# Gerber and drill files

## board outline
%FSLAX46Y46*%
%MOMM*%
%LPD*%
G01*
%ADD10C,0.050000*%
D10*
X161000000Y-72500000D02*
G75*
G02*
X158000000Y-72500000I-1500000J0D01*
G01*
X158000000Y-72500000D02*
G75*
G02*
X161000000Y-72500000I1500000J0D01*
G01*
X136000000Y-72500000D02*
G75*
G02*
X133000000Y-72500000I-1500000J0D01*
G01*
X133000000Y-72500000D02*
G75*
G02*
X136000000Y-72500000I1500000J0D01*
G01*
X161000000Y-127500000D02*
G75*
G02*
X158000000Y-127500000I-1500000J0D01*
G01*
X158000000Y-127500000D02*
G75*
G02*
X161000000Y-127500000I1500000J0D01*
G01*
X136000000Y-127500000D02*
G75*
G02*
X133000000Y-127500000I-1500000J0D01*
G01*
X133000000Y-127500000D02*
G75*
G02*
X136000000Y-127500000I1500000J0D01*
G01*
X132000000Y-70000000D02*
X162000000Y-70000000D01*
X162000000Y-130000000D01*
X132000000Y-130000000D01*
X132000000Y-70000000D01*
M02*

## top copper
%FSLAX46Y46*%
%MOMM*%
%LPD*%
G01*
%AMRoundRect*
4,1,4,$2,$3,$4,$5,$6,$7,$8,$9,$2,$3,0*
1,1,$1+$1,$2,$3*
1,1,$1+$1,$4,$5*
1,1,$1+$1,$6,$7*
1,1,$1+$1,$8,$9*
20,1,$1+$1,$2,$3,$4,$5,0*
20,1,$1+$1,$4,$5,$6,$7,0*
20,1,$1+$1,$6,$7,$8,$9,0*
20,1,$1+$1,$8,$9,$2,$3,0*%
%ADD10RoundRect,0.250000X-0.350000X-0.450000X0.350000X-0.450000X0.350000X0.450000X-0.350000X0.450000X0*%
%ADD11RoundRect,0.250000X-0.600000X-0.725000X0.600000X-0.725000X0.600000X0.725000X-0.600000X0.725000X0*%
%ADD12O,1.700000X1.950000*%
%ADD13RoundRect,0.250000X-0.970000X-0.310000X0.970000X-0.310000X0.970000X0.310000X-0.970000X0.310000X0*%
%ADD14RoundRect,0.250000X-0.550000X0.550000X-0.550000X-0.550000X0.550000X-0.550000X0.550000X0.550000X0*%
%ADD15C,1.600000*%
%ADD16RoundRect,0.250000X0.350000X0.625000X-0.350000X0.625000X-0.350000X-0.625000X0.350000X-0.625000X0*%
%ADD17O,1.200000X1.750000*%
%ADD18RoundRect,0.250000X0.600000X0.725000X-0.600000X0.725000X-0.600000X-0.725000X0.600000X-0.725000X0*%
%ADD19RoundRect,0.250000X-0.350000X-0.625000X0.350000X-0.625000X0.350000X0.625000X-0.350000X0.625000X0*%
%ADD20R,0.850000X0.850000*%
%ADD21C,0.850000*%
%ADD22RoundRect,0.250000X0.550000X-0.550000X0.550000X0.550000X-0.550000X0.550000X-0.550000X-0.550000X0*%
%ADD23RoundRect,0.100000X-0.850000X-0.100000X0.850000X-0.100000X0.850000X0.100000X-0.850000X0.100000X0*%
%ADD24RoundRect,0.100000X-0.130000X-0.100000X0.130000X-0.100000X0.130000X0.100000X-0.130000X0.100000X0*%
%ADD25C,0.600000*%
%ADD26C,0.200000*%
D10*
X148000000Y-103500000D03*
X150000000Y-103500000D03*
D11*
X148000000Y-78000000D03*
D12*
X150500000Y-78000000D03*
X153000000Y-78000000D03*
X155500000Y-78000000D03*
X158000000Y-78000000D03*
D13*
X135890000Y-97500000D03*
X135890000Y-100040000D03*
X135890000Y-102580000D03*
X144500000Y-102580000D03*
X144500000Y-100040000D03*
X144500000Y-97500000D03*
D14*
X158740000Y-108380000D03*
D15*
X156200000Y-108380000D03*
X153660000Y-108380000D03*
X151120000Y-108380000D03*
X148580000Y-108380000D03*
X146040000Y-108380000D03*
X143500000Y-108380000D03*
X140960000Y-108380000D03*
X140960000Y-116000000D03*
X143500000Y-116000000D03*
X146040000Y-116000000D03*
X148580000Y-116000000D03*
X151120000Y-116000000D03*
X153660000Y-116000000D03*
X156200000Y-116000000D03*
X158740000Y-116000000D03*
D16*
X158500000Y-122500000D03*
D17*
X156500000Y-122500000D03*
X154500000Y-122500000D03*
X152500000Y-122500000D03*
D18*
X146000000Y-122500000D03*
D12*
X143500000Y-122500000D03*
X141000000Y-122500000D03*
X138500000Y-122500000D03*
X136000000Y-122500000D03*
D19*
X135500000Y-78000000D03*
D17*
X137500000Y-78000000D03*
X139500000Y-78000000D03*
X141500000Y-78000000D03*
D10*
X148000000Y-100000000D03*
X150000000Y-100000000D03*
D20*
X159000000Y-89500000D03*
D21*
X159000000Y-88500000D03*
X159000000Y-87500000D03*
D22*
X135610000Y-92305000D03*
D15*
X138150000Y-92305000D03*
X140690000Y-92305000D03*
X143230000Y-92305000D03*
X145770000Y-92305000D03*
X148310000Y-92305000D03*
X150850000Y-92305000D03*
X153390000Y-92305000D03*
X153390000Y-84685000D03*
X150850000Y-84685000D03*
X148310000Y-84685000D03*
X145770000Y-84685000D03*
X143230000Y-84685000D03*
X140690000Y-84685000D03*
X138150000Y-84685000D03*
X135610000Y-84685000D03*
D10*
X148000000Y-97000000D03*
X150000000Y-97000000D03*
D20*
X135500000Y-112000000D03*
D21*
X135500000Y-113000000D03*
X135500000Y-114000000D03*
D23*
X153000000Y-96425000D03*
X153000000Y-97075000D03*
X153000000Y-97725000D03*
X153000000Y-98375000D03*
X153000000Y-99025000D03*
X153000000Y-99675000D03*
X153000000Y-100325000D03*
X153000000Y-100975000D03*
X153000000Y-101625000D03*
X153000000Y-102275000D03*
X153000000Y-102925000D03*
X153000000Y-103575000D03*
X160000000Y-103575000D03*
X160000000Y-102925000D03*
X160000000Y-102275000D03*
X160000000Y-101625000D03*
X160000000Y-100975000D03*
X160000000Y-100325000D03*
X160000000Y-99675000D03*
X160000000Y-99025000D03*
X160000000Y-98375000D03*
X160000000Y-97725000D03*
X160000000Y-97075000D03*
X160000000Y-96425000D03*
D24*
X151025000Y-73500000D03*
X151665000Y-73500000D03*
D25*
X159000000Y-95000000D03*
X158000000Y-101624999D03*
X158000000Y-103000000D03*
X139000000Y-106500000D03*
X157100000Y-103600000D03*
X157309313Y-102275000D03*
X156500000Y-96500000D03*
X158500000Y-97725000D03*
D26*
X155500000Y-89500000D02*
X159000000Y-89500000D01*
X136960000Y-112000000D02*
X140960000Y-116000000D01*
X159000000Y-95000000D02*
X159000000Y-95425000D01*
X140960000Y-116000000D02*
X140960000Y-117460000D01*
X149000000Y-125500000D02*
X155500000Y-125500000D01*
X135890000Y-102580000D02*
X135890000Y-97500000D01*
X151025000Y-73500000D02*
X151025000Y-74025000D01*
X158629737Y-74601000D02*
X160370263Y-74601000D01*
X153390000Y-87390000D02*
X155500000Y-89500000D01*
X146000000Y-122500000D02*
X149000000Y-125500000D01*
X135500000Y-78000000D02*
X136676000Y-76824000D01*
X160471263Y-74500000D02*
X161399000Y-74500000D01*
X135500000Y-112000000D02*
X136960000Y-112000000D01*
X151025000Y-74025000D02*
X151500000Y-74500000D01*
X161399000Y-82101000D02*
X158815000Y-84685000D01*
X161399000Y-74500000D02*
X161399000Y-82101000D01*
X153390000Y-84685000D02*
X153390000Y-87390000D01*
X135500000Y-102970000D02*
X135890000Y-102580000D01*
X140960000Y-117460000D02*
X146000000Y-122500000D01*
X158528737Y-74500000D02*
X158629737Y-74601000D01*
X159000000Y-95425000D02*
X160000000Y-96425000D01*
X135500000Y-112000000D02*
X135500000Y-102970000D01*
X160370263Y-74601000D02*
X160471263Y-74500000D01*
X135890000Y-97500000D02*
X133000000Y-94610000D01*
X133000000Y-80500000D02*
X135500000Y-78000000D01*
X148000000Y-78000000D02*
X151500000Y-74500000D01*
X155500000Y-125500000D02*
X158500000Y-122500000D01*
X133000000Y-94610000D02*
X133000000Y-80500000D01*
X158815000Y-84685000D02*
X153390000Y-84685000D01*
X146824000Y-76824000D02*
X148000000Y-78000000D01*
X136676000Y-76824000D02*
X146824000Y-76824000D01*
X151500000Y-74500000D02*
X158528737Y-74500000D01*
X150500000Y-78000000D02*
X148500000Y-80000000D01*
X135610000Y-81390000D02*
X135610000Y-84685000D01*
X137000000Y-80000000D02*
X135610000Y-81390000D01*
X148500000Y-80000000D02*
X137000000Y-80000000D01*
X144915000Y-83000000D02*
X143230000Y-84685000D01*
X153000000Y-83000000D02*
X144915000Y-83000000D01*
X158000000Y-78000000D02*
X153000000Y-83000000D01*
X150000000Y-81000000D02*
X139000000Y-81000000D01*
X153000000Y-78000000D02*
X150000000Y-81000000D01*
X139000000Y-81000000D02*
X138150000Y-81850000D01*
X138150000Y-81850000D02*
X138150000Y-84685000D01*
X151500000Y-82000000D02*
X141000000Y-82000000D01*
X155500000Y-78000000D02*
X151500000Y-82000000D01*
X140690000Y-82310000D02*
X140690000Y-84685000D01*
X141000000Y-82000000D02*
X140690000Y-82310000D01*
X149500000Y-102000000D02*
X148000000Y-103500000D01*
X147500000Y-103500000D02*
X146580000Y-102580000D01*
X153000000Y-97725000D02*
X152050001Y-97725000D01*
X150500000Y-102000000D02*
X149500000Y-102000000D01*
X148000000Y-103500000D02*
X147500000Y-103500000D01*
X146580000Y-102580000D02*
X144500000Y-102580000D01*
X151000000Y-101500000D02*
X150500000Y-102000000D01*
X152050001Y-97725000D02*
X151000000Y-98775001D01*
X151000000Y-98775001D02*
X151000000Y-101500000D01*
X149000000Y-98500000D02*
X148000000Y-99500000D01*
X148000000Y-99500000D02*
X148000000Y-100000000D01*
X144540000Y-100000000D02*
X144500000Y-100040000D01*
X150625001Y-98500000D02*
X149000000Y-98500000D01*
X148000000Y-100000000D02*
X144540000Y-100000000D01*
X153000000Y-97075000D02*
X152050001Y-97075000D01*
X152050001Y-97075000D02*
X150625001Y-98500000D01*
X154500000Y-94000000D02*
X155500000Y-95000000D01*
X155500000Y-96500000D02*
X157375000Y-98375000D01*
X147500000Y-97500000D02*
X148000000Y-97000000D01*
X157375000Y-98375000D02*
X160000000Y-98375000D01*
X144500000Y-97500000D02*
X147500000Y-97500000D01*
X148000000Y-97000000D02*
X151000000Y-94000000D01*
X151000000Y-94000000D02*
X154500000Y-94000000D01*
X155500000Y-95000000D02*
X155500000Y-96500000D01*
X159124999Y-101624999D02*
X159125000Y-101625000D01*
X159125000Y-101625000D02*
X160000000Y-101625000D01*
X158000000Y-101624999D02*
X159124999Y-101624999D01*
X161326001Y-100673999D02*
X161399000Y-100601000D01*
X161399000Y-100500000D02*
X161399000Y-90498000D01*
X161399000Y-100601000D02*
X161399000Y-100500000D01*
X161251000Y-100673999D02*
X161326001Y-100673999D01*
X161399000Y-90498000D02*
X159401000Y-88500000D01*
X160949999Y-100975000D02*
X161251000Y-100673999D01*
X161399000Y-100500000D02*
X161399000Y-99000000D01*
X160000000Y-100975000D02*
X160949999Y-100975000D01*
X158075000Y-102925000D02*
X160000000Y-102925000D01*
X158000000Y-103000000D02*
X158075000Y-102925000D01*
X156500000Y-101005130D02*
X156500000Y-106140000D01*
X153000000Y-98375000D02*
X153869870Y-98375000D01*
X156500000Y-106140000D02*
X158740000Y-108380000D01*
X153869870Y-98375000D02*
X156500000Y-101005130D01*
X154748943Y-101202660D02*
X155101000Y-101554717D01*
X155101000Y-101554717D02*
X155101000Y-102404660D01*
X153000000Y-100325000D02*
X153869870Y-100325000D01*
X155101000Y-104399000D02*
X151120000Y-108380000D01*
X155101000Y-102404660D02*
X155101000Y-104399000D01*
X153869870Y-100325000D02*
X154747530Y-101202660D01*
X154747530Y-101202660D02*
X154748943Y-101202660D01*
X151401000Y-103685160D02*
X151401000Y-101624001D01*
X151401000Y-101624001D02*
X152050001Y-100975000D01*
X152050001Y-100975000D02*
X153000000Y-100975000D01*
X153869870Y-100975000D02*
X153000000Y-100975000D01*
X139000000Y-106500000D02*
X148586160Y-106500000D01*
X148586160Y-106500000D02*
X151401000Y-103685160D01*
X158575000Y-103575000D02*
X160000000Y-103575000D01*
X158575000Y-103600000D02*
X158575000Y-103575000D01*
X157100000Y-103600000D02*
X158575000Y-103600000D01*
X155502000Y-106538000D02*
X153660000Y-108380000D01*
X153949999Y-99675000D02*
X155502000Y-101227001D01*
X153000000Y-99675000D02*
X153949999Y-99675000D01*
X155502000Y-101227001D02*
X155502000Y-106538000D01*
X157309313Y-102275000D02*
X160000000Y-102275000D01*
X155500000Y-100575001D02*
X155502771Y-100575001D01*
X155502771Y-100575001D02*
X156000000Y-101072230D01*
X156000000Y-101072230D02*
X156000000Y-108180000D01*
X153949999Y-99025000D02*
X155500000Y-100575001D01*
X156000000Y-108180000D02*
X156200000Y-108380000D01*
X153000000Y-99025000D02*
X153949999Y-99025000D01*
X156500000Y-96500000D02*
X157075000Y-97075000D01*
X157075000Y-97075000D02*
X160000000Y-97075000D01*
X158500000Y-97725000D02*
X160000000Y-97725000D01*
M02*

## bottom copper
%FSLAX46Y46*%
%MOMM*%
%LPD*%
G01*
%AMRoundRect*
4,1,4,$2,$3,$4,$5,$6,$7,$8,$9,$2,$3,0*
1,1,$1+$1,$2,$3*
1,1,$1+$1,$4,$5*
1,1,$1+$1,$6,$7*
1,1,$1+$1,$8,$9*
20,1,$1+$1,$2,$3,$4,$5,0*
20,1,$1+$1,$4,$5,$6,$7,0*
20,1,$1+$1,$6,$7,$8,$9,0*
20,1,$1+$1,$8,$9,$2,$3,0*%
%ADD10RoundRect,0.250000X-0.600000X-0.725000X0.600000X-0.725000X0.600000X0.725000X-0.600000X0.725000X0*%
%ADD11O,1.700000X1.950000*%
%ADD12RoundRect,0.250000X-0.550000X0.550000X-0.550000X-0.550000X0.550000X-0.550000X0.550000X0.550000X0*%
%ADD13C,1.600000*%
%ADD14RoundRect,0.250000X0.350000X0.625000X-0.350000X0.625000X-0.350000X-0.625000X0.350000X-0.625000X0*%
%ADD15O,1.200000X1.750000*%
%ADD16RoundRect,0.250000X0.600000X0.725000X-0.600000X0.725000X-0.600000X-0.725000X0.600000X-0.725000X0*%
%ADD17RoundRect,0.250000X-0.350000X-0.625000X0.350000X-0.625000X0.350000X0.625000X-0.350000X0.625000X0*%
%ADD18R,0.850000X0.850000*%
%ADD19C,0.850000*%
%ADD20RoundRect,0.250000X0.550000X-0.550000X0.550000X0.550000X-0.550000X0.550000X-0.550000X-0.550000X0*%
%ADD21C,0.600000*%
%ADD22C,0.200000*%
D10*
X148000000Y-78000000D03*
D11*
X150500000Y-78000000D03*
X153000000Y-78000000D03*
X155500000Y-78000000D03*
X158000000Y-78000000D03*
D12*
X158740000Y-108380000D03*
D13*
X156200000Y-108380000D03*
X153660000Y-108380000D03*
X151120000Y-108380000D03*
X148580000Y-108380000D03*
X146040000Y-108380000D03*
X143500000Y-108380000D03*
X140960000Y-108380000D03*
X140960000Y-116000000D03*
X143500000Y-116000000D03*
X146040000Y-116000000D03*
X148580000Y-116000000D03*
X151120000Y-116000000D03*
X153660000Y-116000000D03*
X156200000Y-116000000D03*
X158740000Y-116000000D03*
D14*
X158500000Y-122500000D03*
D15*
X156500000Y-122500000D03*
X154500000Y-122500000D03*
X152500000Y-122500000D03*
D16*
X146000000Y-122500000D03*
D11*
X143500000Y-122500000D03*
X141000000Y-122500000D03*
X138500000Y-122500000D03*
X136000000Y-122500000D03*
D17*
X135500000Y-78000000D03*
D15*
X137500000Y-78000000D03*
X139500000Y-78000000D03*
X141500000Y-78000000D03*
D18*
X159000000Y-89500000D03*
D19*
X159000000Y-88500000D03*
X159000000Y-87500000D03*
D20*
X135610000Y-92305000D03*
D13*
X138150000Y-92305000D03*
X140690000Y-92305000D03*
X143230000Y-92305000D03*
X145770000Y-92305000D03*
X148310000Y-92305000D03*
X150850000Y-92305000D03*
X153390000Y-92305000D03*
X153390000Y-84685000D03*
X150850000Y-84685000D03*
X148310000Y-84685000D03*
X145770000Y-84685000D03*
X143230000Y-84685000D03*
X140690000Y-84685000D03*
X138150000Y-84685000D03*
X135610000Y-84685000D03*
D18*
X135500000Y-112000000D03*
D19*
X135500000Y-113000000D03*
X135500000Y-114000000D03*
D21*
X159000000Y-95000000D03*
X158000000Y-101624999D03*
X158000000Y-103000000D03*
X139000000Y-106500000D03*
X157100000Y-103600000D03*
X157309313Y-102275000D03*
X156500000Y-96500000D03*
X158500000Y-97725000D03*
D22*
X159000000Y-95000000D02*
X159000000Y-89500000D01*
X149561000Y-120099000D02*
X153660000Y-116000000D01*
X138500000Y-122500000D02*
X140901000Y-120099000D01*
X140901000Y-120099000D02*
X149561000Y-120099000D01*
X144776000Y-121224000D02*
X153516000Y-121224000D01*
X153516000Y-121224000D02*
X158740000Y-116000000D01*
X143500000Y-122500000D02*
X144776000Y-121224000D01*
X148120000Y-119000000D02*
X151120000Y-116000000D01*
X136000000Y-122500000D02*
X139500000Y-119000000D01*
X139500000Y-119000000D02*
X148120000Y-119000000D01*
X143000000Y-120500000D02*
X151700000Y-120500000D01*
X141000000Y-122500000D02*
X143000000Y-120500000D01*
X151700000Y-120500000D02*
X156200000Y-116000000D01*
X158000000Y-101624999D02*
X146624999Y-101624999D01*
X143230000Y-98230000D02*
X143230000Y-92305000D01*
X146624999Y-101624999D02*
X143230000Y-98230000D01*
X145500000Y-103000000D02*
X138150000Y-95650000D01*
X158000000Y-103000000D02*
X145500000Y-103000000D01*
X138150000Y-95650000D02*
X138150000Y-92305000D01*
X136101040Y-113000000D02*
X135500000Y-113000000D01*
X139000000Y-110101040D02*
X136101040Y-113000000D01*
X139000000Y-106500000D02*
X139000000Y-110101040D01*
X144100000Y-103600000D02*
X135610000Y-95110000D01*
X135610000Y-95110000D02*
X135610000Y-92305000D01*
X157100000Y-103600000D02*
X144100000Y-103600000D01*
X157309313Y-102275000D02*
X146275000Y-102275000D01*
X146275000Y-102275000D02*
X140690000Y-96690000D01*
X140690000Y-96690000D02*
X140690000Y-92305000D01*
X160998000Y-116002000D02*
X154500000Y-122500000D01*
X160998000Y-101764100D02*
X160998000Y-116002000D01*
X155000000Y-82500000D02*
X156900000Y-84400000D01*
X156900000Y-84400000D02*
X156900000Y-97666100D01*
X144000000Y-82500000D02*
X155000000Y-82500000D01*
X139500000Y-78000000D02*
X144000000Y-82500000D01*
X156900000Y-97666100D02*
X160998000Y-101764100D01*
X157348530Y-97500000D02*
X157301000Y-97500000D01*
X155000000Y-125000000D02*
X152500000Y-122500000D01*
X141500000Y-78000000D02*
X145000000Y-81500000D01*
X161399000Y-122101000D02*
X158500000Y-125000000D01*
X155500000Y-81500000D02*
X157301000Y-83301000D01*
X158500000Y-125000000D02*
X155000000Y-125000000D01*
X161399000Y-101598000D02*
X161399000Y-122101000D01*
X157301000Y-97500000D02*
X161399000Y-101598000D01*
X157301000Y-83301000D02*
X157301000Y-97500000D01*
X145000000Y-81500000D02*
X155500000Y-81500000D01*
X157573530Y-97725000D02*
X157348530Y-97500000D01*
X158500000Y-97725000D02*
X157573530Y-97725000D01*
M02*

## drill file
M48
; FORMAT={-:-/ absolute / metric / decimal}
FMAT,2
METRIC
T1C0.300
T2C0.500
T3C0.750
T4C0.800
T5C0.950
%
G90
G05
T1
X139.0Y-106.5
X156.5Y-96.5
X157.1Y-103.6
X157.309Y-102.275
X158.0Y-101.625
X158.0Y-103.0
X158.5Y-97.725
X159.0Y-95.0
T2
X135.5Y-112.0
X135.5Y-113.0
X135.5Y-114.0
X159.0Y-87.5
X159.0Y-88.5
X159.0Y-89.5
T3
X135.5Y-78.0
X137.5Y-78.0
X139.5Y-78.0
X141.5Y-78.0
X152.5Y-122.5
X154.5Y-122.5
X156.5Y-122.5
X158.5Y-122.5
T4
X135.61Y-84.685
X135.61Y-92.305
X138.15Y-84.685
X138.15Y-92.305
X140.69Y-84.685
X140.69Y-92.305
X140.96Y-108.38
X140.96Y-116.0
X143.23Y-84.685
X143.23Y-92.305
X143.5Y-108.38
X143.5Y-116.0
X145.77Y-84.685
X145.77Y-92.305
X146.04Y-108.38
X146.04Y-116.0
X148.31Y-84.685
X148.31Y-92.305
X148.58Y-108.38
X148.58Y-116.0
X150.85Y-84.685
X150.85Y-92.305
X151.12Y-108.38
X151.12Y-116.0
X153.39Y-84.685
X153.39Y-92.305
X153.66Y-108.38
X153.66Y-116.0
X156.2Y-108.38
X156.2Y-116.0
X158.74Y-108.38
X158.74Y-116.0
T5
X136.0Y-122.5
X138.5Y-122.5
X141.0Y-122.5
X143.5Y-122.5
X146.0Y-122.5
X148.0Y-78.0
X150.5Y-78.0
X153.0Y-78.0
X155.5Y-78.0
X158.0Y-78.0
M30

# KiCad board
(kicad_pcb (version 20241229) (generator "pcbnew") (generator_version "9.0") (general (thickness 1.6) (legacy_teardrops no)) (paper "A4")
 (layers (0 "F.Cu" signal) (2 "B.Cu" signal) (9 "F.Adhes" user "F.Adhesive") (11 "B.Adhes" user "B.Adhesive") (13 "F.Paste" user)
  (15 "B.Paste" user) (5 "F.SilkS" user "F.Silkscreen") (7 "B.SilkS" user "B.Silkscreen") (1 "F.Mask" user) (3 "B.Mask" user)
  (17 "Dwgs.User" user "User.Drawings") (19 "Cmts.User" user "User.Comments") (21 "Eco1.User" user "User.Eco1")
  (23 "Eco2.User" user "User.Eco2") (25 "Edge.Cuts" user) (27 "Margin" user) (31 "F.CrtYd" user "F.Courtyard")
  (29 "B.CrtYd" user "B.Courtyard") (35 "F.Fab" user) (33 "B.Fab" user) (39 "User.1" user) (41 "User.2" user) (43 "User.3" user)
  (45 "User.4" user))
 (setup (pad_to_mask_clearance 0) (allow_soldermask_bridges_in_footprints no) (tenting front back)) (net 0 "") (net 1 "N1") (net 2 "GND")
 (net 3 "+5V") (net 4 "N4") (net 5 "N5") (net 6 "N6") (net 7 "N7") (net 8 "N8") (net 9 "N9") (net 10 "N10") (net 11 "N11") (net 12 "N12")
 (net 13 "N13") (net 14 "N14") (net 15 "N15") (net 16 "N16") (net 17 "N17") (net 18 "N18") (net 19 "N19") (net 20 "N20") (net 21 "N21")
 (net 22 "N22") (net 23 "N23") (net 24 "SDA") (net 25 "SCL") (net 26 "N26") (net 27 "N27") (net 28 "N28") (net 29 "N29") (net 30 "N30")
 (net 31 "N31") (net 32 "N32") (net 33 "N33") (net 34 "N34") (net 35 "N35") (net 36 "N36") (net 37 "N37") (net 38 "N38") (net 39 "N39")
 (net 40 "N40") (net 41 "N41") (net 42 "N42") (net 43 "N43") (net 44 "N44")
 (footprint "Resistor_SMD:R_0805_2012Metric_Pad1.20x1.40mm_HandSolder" (layer "F.Cu") (at 149 103.5)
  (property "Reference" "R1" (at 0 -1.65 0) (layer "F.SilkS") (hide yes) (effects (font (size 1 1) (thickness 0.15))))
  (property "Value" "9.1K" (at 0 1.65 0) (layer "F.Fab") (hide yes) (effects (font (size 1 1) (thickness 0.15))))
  (pad "1" smd roundrect (at -1 0) (size 1.2 1.4) (layers "F.Cu" "F.Mask" "F.Paste") (roundrect_rratio 0.208333) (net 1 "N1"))
  (pad "2" smd roundrect (at 1 0) (size 1.2 1.4) (layers "F.Cu" "F.Mask" "F.Paste") (roundrect_rratio 0.208333) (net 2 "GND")))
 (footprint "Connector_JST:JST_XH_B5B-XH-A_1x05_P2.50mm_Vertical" (layer "F.Cu") (at 148 78)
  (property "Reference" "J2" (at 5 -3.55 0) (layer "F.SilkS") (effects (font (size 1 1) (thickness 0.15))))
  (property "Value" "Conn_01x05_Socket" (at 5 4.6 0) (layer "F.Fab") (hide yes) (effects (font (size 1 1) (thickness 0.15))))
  (pad "1" thru_hole roundrect (at 0 0) (size 1.7 1.95) (drill 0.95) (layers "*.Cu" "*.Mask") (remove_unused_layers no)
   (roundrect_rratio 0.147059) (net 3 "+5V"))
  (pad "2" thru_hole oval (at 2.5 0) (size 1.7 1.95) (drill 0.95) (layers "*.Cu" "*.Mask") (remove_unused_layers no) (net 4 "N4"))
  (pad "3" thru_hole oval (at 5 0) (size 1.7 1.95) (drill 0.95) (layers "*.Cu" "*.Mask") (remove_unused_layers no) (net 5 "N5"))
  (pad "4" thru_hole oval (at 7.5 0) (size 1.7 1.95) (drill 0.95) (layers "*.Cu" "*.Mask") (remove_unused_layers no) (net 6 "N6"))
  (pad "5" thru_hole oval (at 10 0) (size 1.7 1.95) (drill 0.95) (layers "*.Cu" "*.Mask") (remove_unused_layers no) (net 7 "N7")))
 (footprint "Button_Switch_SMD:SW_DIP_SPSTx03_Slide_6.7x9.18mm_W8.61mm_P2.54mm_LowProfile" (layer "F.Cu") (at 140.195 100.04)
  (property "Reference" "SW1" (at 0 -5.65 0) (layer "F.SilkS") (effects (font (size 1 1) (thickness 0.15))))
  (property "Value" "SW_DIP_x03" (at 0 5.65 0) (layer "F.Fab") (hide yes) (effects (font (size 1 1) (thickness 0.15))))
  (pad "1" smd roundrect (at -4.305 -2.54) (size 2.44 1.12) (layers "F.Cu" "F.Mask" "F.Paste") (roundrect_rratio 0.223214) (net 3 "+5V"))
  (pad "2" smd roundrect (at -4.305 0) (size 2.44 1.12) (layers "F.Cu" "F.Mask" "F.Paste") (roundrect_rratio 0.223214) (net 3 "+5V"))
  (pad "3" smd roundrect (at -4.305 2.54) (size 2.44 1.12) (layers "F.Cu" "F.Mask" "F.Paste") (roundrect_rratio 0.223214) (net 3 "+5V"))
  (pad "4" smd roundrect (at 4.305 2.54) (size 2.44 1.12) (layers "F.Cu" "F.Mask" "F.Paste") (roundrect_rratio 0.223214) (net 1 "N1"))
  (pad "5" smd roundrect (at 4.305 0) (size 2.44 1.12) (layers "F.Cu" "F.Mask" "F.Paste") (roundrect_rratio 0.223214) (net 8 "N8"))
  (pad "6" smd roundrect (at 4.305 -2.54) (size 2.44 1.12) (layers "F.Cu" "F.Mask" "F.Paste") (roundrect_rratio 0.223214) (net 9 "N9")))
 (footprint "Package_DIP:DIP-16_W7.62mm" (layer "F.Cu") (at 158.74 108.38 -90)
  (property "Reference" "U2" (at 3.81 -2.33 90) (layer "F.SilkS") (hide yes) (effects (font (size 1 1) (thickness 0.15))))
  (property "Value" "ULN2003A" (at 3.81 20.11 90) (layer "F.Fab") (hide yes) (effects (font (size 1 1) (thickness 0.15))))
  (pad "1" thru_hole roundrect (at 0 0 270) (size 1.6 1.6) (drill 0.8) (layers "*.Cu" "*.Mask") (remove_unused_layers no)
   (roundrect_rratio 0.15625) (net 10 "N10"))
  (pad "2" thru_hole circle (at 0 2.54 270) (size 1.6 1.6) (drill 0.8) (layers "*.Cu" "*.Mask") (remove_unused_layers no) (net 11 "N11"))
  (pad "3" thru_hole circle (at 0 5.08 270) (size 1.6 1.6) (drill 0.8) (layers "*.Cu" "*.Mask") (remove_unused_layers no) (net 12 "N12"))
  (pad "4" thru_hole circle (at 0 7.62 270) (size 1.6 1.6) (drill 0.8) (layers "*.Cu" "*.Mask") (remove_unused_layers no) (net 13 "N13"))
  (pad "5" thru_hole circle (at 0 10.16 270) (size 1.6 1.6) (drill 0.8) (layers "*.Cu" "*.Mask") (remove_unused_layers no) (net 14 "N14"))
  (pad "6" thru_hole circle (at 0 12.7 270) (size 1.6 1.6) (drill 0.8) (layers "*.Cu" "*.Mask") (remove_unused_layers no) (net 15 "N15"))
  (pad "7" thru_hole circle (at 0 15.24 270) (size 1.6 1.6) (drill 0.8) (layers "*.Cu" "*.Mask") (remove_unused_layers no) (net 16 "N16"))
  (pad "8" thru_hole circle (at 0 17.78 270) (size 1.6 1.6) (drill 0.8) (layers "*.Cu" "*.Mask") (remove_unused_layers no) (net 2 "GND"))
  (pad "9" thru_hole circle (at 7.62 17.78 270) (size 1.6 1.6) (drill 0.8) (layers "*.Cu" "*.Mask") (remove_unused_layers no) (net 3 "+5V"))
  (pad "10" thru_hole circle (at 7.62 15.24 270) (size 1.6 1.6) (drill 0.8) (layers "*.Cu" "*.Mask") (remove_unused_layers no)
   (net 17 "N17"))
  (pad "11" thru_hole circle (at 7.62 12.7 270) (size 1.6 1.6) (drill 0.8) (layers "*.Cu" "*.Mask") (remove_unused_layers no) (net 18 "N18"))
  (pad "12" thru_hole circle (at 7.62 10.16 270) (size 1.6 1.6) (drill 0.8) (layers "*.Cu" "*.Mask") (remove_unused_layers no)
   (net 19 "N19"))
  (pad "13" thru_hole circle (at 7.62 7.62 270) (size 1.6 1.6) (drill 0.8) (layers "*.Cu" "*.Mask") (remove_unused_layers no) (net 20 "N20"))
  (pad "14" thru_hole circle (at 7.62 5.08 270) (size 1.6 1.6) (drill 0.8) (layers "*.Cu" "*.Mask") (remove_unused_layers no) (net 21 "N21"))
  (pad "15" thru_hole circle (at 7.62 2.54 270) (size 1.6 1.6) (drill 0.8) (layers "*.Cu" "*.Mask") (remove_unused_layers no) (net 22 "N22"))
  (pad "16" thru_hole circle (at 7.62 0 270) (size 1.6 1.6) (drill 0.8) (layers "*.Cu" "*.Mask") (remove_unused_layers no) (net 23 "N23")))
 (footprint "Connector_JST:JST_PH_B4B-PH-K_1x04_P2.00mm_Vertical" (layer "F.Cu") (at 158.5 122.5 180)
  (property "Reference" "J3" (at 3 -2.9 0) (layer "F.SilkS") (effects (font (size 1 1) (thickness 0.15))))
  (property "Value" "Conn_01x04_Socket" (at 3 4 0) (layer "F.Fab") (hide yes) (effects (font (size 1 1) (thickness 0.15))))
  (pad "1" thru_hole roundrect (at 0 0 180) (size 1.2 1.75) (drill 0.75) (layers "*.Cu" "*.Mask") (remove_unused_layers no)
   (roundrect_rratio 0.208333) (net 3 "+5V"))
  (pad "2" thru_hole oval (at 2 0 180) (size 1.2 1.75) (drill 0.75) (layers "*.Cu" "*.Mask") (remove_unused_layers no) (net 2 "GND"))
  (pad "3" thru_hole oval (at 4 0 180) (size 1.2 1.75) (drill 0.75) (layers "*.Cu" "*.Mask") (remove_unused_layers no) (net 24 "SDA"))
  (pad "4" thru_hole oval (at 6 0 180) (size 1.2 1.75) (drill 0.75) (layers "*.Cu" "*.Mask") (remove_unused_layers no) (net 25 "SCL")))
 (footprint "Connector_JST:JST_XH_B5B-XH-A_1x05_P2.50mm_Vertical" (layer "F.Cu") (at 146 122.5 180)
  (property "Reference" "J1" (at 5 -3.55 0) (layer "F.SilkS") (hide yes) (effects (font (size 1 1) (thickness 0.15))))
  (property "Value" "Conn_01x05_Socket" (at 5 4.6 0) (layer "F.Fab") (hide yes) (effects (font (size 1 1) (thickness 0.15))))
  (pad "1" thru_hole roundrect (at 0 0 180) (size 1.7 1.95) (drill 0.95) (layers "*.Cu" "*.Mask") (remove_unused_layers no)
   (roundrect_rratio 0.147059) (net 3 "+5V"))
  (pad "2" thru_hole oval (at 2.5 0 180) (size 1.7 1.95) (drill 0.95) (layers "*.Cu" "*.Mask") (remove_unused_layers no) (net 23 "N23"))
  (pad "3" thru_hole oval (at 5 0 180) (size 1.7 1.95) (drill 0.95) (layers "*.Cu" "*.Mask") (remove_unused_layers no) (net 22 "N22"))
  (pad "4" thru_hole oval (at 7.5 0 180) (size 1.7 1.95) (drill 0.95) (layers "*.Cu" "*.Mask") (remove_unused_layers no) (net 21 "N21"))
  (pad "5" thru_hole oval (at 10 0 180) (size 1.7 1.95) (drill 0.95) (layers "*.Cu" "*.Mask") (remove_unused_layers no) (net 20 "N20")))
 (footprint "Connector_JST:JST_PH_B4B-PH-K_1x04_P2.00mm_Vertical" (layer "F.Cu") (at 135.5 78)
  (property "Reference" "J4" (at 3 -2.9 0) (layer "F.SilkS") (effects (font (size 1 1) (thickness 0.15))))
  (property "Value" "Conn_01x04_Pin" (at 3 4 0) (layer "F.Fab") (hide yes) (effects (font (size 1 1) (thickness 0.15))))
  (pad "1" thru_hole roundrect (at 0 0) (size 1.2 1.75) (drill 0.75) (layers "*.Cu" "*.Mask") (remove_unused_layers no)
   (roundrect_rratio 0.208333) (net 3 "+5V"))
  (pad "2" thru_hole oval (at 2 0) (size 1.2 1.75) (drill 0.75) (layers "*.Cu" "*.Mask") (remove_unused_layers no) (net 2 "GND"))
  (pad "3" thru_hole oval (at 4 0) (size 1.2 1.75) (drill 0.75) (layers "*.Cu" "*.Mask") (remove_unused_layers no) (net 24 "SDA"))
  (pad "4" thru_hole oval (at 6 0) (size 1.2 1.75) (drill 0.75) (layers "*.Cu" "*.Mask") (remove_unused_layers no) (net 25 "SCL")))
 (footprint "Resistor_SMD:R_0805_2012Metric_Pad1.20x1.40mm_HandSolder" (layer "F.Cu") (at 149 100)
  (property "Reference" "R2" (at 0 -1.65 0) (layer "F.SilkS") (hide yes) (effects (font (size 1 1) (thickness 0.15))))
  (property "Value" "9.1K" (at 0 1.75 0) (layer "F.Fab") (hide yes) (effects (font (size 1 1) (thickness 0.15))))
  (pad "1" smd roundrect (at -1 0) (size 1.2 1.4) (layers "F.Cu" "F.Mask" "F.Paste") (roundrect_rratio 0.208333) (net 8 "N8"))
  (pad "2" smd roundrect (at 1 0) (size 1.2 1.4) (layers "F.Cu" "F.Mask" "F.Paste") (roundrect_rratio 0.208333) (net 2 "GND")))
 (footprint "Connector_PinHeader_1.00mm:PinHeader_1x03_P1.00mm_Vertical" (layer "F.Cu") (at 159 89.5 180)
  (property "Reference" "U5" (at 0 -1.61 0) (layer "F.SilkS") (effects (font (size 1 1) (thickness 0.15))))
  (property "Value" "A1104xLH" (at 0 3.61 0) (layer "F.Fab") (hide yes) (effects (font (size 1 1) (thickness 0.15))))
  (pad "1" thru_hole rect (at 0 0 180) (size 0.85 0.85) (drill 0.5) (layers "*.Cu" "*.Mask") (remove_unused_layers no) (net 3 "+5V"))
  (pad "2" thru_hole circle (at 0 1 180) (size 0.85 0.85) (drill 0.5) (layers "*.Cu" "*.Mask") (remove_unused_layers no) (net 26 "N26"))
  (pad "3" thru_hole circle (at 0 2 180) (size 0.85 0.85) (drill 0.5) (layers "*.Cu" "*.Mask") (remove_unused_layers no) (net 2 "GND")))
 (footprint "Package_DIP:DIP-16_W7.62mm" (layer "F.Cu") (at 135.61 92.305 90)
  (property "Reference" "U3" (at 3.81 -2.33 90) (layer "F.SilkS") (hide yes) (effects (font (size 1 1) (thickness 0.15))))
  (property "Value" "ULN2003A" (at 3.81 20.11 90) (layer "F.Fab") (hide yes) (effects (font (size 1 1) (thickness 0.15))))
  (pad "1" thru_hole roundrect (at 0 0 90) (size 1.6 1.6) (drill 0.8) (layers "*.Cu" "*.Mask") (remove_unused_layers no)
   (roundrect_rratio 0.15625) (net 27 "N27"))
  (pad "2" thru_hole circle (at 0 2.54 90) (size 1.6 1.6) (drill 0.8) (layers "*.Cu" "*.Mask") (remove_unused_layers no) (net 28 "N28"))
  (pad "3" thru_hole circle (at 0 5.08 90) (size 1.6 1.6) (drill 0.8) (layers "*.Cu" "*.Mask") (remove_unused_layers no) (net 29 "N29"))
  (pad "4" thru_hole circle (at 0 7.62 90) (size 1.6 1.6) (drill 0.8) (layers "*.Cu" "*.Mask") (remove_unused_layers no) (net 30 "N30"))
  (pad "5" thru_hole circle (at 0 10.16 90) (size 1.6 1.6) (drill 0.8) (layers "*.Cu" "*.Mask") (remove_unused_layers no) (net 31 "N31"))
  (pad "6" thru_hole circle (at 0 12.7 90) (size 1.6 1.6) (drill 0.8) (layers "*.Cu" "*.Mask") (remove_unused_layers no) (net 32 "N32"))
  (pad "7" thru_hole circle (at 0 15.24 90) (size 1.6 1.6) (drill 0.8) (layers "*.Cu" "*.Mask") (remove_unused_layers no) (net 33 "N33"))
  (pad "8" thru_hole circle (at 0 17.78 90) (size 1.6 1.6) (drill 0.8) (layers "*.Cu" "*.Mask") (remove_unused_layers no) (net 2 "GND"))
  (pad "9" thru_hole circle (at 7.62 17.78 90) (size 1.6 1.6) (drill 0.8) (layers "*.Cu" "*.Mask") (remove_unused_layers no) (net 3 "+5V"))
  (pad "10" thru_hole circle (at 7.62 15.24 90) (size 1.6 1.6) (drill 0.8) (layers "*.Cu" "*.Mask") (remove_unused_layers no) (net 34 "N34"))
  (pad "11" thru_hole circle (at 7.62 12.7 90) (size 1.6 1.6) (drill 0.8) (layers "*.Cu" "*.Mask") (remove_unused_layers no) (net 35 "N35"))
  (pad "12" thru_hole circle (at 7.62 10.16 90) (size 1.6 1.6) (drill 0.8) (layers "*.Cu" "*.Mask") (remove_unused_layers no) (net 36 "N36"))
  (pad "13" thru_hole circle (at 7.62 7.62 90) (size 1.6 1.6) (drill 0.8) (layers "*.Cu" "*.Mask") (remove_unused_layers no) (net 7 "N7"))
  (pad "14" thru_hole circle (at 7.62 5.08 90) (size 1.6 1.6) (drill 0.8) (layers "*.Cu" "*.Mask") (remove_unused_layers no) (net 6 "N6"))
  (pad "15" thru_hole circle (at 7.62 2.54 90) (size 1.6 1.6) (drill 0.8) (layers "*.Cu" "*.Mask") (remove_unused_layers no) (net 5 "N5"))
  (pad "16" thru_hole circle (at 7.62 0 90) (size 1.6 1.6) (drill 0.8) (layers "*.Cu" "*.Mask") (remove_unused_layers no) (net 4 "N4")))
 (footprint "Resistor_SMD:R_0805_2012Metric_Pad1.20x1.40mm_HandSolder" (layer "F.Cu") (at 149 97)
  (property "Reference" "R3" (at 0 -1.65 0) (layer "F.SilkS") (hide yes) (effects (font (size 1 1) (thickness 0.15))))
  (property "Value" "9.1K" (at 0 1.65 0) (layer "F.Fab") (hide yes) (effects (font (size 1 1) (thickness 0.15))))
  (pad "1" smd roundrect (at -1 0) (size 1.2 1.4) (layers "F.Cu" "F.Mask" "F.Paste") (roundrect_rratio 0.208333) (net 9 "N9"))
  (pad "2" smd roundrect (at 1 0) (size 1.2 1.4) (layers "F.Cu" "F.Mask" "F.Paste") (roundrect_rratio 0.208333) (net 2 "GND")))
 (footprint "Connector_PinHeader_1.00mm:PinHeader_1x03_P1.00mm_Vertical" (layer "F.Cu") (at 135.5 112)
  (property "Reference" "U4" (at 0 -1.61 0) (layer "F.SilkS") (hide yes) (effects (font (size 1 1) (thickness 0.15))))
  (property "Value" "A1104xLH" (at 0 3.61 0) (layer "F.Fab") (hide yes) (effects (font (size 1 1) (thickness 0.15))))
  (pad "1" thru_hole rect (at 0 0) (size 0.85 0.85) (drill 0.5) (layers "*.Cu" "*.Mask") (remove_unused_layers no) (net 3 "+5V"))
  (pad "2" thru_hole circle (at 0 1) (size 0.85 0.85) (drill 0.5) (layers "*.Cu" "*.Mask") (remove_unused_layers no) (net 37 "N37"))
  (pad "3" thru_hole circle (at 0 2) (size 0.85 0.85) (drill 0.5) (layers "*.Cu" "*.Mask") (remove_unused_layers no) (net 2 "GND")))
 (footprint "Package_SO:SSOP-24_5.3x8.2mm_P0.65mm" (layer "F.Cu") (at 156.5 100)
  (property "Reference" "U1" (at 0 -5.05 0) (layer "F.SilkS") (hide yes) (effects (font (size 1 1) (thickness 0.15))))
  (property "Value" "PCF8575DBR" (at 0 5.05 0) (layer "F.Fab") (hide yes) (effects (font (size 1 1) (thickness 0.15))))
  (pad "1" smd roundrect (at -3.5 -3.575) (size 1.9 0.4) (layers "F.Cu" "F.Mask" "F.Paste") (roundrect_rratio 0.25) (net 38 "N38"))
  (pad "2" smd roundrect (at -3.5 -2.925) (size 1.9 0.4) (layers "F.Cu" "F.Mask" "F.Paste") (roundrect_rratio 0.25) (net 8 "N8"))
  (pad "3" smd roundrect (at -3.5 -2.275) (size 1.9 0.4) (layers "F.Cu" "F.Mask" "F.Paste") (roundrect_rratio 0.25) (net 1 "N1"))
  (pad "4" smd roundrect (at -3.5 -1.625) (size 1.9 0.4) (layers "F.Cu" "F.Mask" "F.Paste") (roundrect_rratio 0.25) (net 10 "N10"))
  (pad "5" smd roundrect (at -3.5 -0.975) (size 1.9 0.4) (layers "F.Cu" "F.Mask" "F.Paste") (roundrect_rratio 0.25) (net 11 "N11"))
  (pad "6" smd roundrect (at -3.5 -0.325) (size 1.9 0.4) (layers "F.Cu" "F.Mask" "F.Paste") (roundrect_rratio 0.25) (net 12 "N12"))
  (pad "7" smd roundrect (at -3.5 0.325) (size 1.9 0.4) (layers "F.Cu" "F.Mask" "F.Paste") (roundrect_rratio 0.25) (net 13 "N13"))
  (pad "8" smd roundrect (at -3.5 0.975) (size 1.9 0.4) (layers "F.Cu" "F.Mask" "F.Paste") (roundrect_rratio 0.25) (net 37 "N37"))
  (pad "9" smd roundrect (at -3.5 1.625) (size 1.9 0.4) (layers "F.Cu" "F.Mask" "F.Paste") (roundrect_rratio 0.25) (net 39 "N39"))
  (pad "10" smd roundrect (at -3.5 2.275) (size 1.9 0.4) (layers "F.Cu" "F.Mask" "F.Paste") (roundrect_rratio 0.25) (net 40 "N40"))
  (pad "11" smd roundrect (at -3.5 2.925) (size 1.9 0.4) (layers "F.Cu" "F.Mask" "F.Paste") (roundrect_rratio 0.25) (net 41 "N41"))
  (pad "12" smd roundrect (at -3.5 3.575) (size 1.9 0.4) (layers "F.Cu" "F.Mask" "F.Paste") (roundrect_rratio 0.25) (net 2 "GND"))
  (pad "13" smd roundrect (at 3.5 3.575) (size 1.9 0.4) (layers "F.Cu" "F.Mask" "F.Paste") (roundrect_rratio 0.25) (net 27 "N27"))
  (pad "14" smd roundrect (at 3.5 2.925) (size 1.9 0.4) (layers "F.Cu" "F.Mask" "F.Paste") (roundrect_rratio 0.25) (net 28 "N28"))
  (pad "15" smd roundrect (at 3.5 2.275) (size 1.9 0.4) (layers "F.Cu" "F.Mask" "F.Paste") (roundrect_rratio 0.25) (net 29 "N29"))
  (pad "16" smd roundrect (at 3.5 1.625) (size 1.9 0.4) (layers "F.Cu" "F.Mask" "F.Paste") (roundrect_rratio 0.25) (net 30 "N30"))
  (pad "17" smd roundrect (at 3.5 0.975) (size 1.9 0.4) (layers "F.Cu" "F.Mask" "F.Paste") (roundrect_rratio 0.25) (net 26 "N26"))
  (pad "18" smd roundrect (at 3.5 0.325) (size 1.9 0.4) (layers "F.Cu" "F.Mask" "F.Paste") (roundrect_rratio 0.25) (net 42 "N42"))
  (pad "19" smd roundrect (at 3.5 -0.325) (size 1.9 0.4) (layers "F.Cu" "F.Mask" "F.Paste") (roundrect_rratio 0.25) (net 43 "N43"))
  (pad "20" smd roundrect (at 3.5 -0.975) (size 1.9 0.4) (layers "F.Cu" "F.Mask" "F.Paste") (roundrect_rratio 0.25) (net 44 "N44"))
  (pad "21" smd roundrect (at 3.5 -1.625) (size 1.9 0.4) (layers "F.Cu" "F.Mask" "F.Paste") (roundrect_rratio 0.25) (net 9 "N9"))
  (pad "22" smd roundrect (at 3.5 -2.275) (size 1.9 0.4) (layers "F.Cu" "F.Mask" "F.Paste") (roundrect_rratio 0.25) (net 25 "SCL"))
  (pad "23" smd roundrect (at 3.5 -2.925) (size 1.9 0.4) (layers "F.Cu" "F.Mask" "F.Paste") (roundrect_rratio 0.25) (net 24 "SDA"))
  (pad "24" smd roundrect (at 3.5 -3.575) (size 1.9 0.4) (layers "F.Cu" "F.Mask" "F.Paste") (roundrect_rratio 0.25) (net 3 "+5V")))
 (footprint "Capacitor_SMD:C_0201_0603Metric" (layer "F.Cu") (at 151.345 73.5)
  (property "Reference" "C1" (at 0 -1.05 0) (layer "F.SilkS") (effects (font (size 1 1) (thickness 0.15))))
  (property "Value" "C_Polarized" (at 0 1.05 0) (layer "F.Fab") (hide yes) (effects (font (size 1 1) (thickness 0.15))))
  (pad "" smd roundrect (at -0.345 0) (size 0.318 0.36) (layers "F.Paste") (roundrect_rratio 0.25))
  (pad "" smd roundrect (at 0.345 0) (size 0.318 0.36) (layers "F.Paste") (roundrect_rratio 0.25))
  (pad "1" smd roundrect (at -0.32 0) (size 0.46 0.4) (layers "F.Cu" "F.Mask") (roundrect_rratio 0.25) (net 3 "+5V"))
  (pad "2" smd roundrect (at 0.32 0) (size 0.46 0.4) (layers "F.Cu" "F.Mask") (roundrect_rratio 0.25) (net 2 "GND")))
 (gr_circle (center 159.5 72.5) (end 161 72.5) (stroke (width 0.05) (type default)) (fill no) (layer "Edge.Cuts"))
 (gr_circle (center 134.5 72.5) (end 136 72.5) (stroke (width 0.05) (type default)) (fill no) (layer "Edge.Cuts"))
 (gr_circle (center 159.5 127.5) (end 161 127.5) (stroke (width 0.05) (type default)) (fill no) (layer "Edge.Cuts"))
 (gr_circle (center 134.5 127.5) (end 136 127.5) (stroke (width 0.05) (type default)) (fill no) (layer "Edge.Cuts"))
 (gr_rect (start 132 70) (end 162 130) (stroke (width 0.05) (type solid)) (fill no) (layer "Edge.Cuts"))
 (segment (start 155.5 89.5) (end 159 89.5) (width 0.2) (layer "F.Cu") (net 3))
 (segment (start 136.96 112) (end 140.96 116) (width 0.2) (layer "F.Cu") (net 3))
 (segment (start 159 95) (end 159 95.425) (width 0.2) (layer "F.Cu") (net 3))
 (segment (start 140.96 116) (end 140.96 117.46) (width 0.2) (layer "F.Cu") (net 3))
 (segment (start 149 125.5) (end 155.5 125.5) (width 0.2) (layer "F.Cu") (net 3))
 (segment (start 135.89 102.58) (end 135.89 97.5) (width 0.2) (layer "F.Cu") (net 3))
 (segment (start 151.025 73.5) (end 151.025 74.025) (width 0.2) (layer "F.Cu") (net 3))
 (segment (start 158.629737 74.601) (end 160.370263 74.601) (width 0.2) (layer "F.Cu") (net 3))
 (segment (start 153.39 87.39) (end 155.5 89.5) (width 0.2) (layer "F.Cu") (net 3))
 (segment (start 146 122.5) (end 149 125.5) (width 0.2) (layer "F.Cu") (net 3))
 (segment (start 135.5 78) (end 136.676 76.824) (width 0.2) (layer "F.Cu") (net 3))
 (segment (start 160.471263 74.5) (end 161.399 74.5) (width 0.2) (layer "F.Cu") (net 3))
 (segment (start 135.5 112) (end 136.96 112) (width 0.2) (layer "F.Cu") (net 3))
 (segment (start 151.025 74.025) (end 151.5 74.5) (width 0.2) (layer "F.Cu") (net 3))
 (segment (start 161.399 82.101) (end 158.815 84.685) (width 0.2) (layer "F.Cu") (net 3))
 (segment (start 161.399 74.5) (end 161.399 82.101) (width 0.2) (layer "F.Cu") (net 3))
 (segment (start 153.39 84.685) (end 153.39 87.39) (width 0.2) (layer "F.Cu") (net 3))
 (segment (start 135.5 102.97) (end 135.89 102.58) (width 0.2) (layer "F.Cu") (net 3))
 (segment (start 140.96 117.46) (end 146 122.5) (width 0.2) (layer "F.Cu") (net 3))
 (segment (start 158.528737 74.5) (end 158.629737 74.601) (width 0.2) (layer "F.Cu") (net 3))
 (segment (start 159 95.425) (end 160 96.425) (width 0.2) (layer "F.Cu") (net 3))
 (segment (start 135.5 112) (end 135.5 102.97) (width 0.2) (layer "F.Cu") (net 3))
 (segment (start 160.370263 74.601) (end 160.471263 74.5) (width 0.2) (layer "F.Cu") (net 3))
 (segment (start 135.89 97.5) (end 133 94.61) (width 0.2) (layer "F.Cu") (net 3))
 (segment (start 133 80.5) (end 135.5 78) (width 0.2) (layer "F.Cu") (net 3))
 (segment (start 148 78) (end 151.5 74.5) (width 0.2) (layer "F.Cu") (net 3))
 (segment (start 155.5 125.5) (end 158.5 122.5) (width 0.2) (layer "F.Cu") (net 3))
 (segment (start 133 94.61) (end 133 80.5) (width 0.2) (layer "F.Cu") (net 3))
 (segment (start 158.815 84.685) (end 153.39 84.685) (width 0.2) (layer "F.Cu") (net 3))
 (segment (start 146.824 76.824) (end 148 78) (width 0.2) (layer "F.Cu") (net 3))
 (segment (start 136.676 76.824) (end 146.824 76.824) (width 0.2) (layer "F.Cu") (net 3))
 (segment (start 151.5 74.5) (end 158.528737 74.5) (width 0.2) (layer "F.Cu") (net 3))
 (via (at 159 95) (size 0.6) (drill 0.3) (layers "F.Cu" "B.Cu") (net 3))
 (segment (start 159 95) (end 159 89.5) (width 0.2) (layer "B.Cu") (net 3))
 (segment (start 149.561 120.099) (end 153.66 116) (width 0.2) (layer "B.Cu") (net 21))
 (segment (start 138.5 122.5) (end 140.901 120.099) (width 0.2) (layer "B.Cu") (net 21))
 (segment (start 140.901 120.099) (end 149.561 120.099) (width 0.2) (layer "B.Cu") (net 21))
 (segment (start 144.776 121.224) (end 153.516 121.224) (width 0.2) (layer "B.Cu") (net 23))
 (segment (start 153.516 121.224) (end 158.74 116) (width 0.2) (layer "B.Cu") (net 23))
 (segment (start 143.5 122.5) (end 144.776 121.224) (width 0.2) (layer "B.Cu") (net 23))
 (segment (start 148.12 119) (end 151.12 116) (width 0.2) (layer "B.Cu") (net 20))
 (segment (start 136 122.5) (end 139.5 119) (width 0.2) (layer "B.Cu") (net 20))
 (segment (start 139.5 119) (end 148.12 119) (width 0.2) (layer "B.Cu") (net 20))
 (segment (start 143 120.5) (end 151.7 120.5) (width 0.2) (layer "B.Cu") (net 22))
 (segment (start 141 122.5) (end 143 120.5) (width 0.2) (layer "B.Cu") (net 22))
 (segment (start 151.7 120.5) (end 156.2 116) (width 0.2) (layer "B.Cu") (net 22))
 (segment (start 150.5 78) (end 148.5 80) (width 0.2) (layer "F.Cu") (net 4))
 (segment (start 135.61 81.39) (end 135.61 84.685) (width 0.2) (layer "F.Cu") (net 4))
 (segment (start 137 80) (end 135.61 81.39) (width 0.2) (layer "F.Cu") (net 4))
 (segment (start 148.5 80) (end 137 80) (width 0.2) (layer "F.Cu") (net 4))
 (segment (start 144.915 83) (end 143.23 84.685) (width 0.2) (layer "F.Cu") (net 7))
 (segment (start 153 83) (end 144.915 83) (width 0.2) (layer "F.Cu") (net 7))
 (segment (start 158 78) (end 153 83) (width 0.2) (layer "F.Cu") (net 7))
 (segment (start 150 81) (end 139 81) (width 0.2) (layer "F.Cu") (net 5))
 (segment (start 153 78) (end 150 81) (width 0.2) (layer "F.Cu") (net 5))
 (segment (start 139 81) (end 138.15 81.85) (width 0.2) (layer "F.Cu") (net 5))
 (segment (start 138.15 81.85) (end 138.15 84.685) (width 0.2) (layer "F.Cu") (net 5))
 (segment (start 151.5 82) (end 141 82) (width 0.2) (layer "F.Cu") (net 6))
 (segment (start 155.5 78) (end 151.5 82) (width 0.2) (layer "F.Cu") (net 6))
 (segment (start 140.69 82.31) (end 140.69 84.685) (width 0.2) (layer "F.Cu") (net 6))
 (segment (start 141 82) (end 140.69 82.31) (width 0.2) (layer "F.Cu") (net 6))
 (segment (start 149.5 102) (end 148 103.5) (width 0.2) (layer "F.Cu") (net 1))
 (segment (start 147.5 103.5) (end 146.58 102.58) (width 0.2) (layer "F.Cu") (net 1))
 (segment (start 153 97.725) (end 152.050001 97.725) (width 0.2) (layer "F.Cu") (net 1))
 (segment (start 150.5 102) (end 149.5 102) (width 0.2) (layer "F.Cu") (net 1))
 (segment (start 148 103.5) (end 147.5 103.5) (width 0.2) (layer "F.Cu") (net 1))
 (segment (start 146.58 102.58) (end 144.5 102.58) (width 0.2) (layer "F.Cu") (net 1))
 (segment (start 151 101.5) (end 150.5 102) (width 0.2) (layer "F.Cu") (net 1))
 (segment (start 152.050001 97.725) (end 151 98.775001) (width 0.2) (layer "F.Cu") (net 1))
 (segment (start 151 98.775001) (end 151 101.5) (width 0.2) (layer "F.Cu") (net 1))
 (segment (start 149 98.5) (end 148 99.5) (width 0.2) (layer "F.Cu") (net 8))
 (segment (start 148 99.5) (end 148 100) (width 0.2) (layer "F.Cu") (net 8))
 (segment (start 144.54 100) (end 144.5 100.04) (width 0.2) (layer "F.Cu") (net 8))
 (segment (start 150.625001 98.5) (end 149 98.5) (width 0.2) (layer "F.Cu") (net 8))
 (segment (start 148 100) (end 144.54 100) (width 0.2) (layer "F.Cu") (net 8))
 (segment (start 153 97.075) (end 152.050001 97.075) (width 0.2) (layer "F.Cu") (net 8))
 (segment (start 152.050001 97.075) (end 150.625001 98.5) (width 0.2) (layer "F.Cu") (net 8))
 (segment (start 154.5 94) (end 155.5 95) (width 0.2) (layer "F.Cu") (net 9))
 (segment (start 155.5 96.5) (end 157.375 98.375) (width 0.2) (layer "F.Cu") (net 9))
 (segment (start 147.5 97.5) (end 148 97) (width 0.2) (layer "F.Cu") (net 9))
 (segment (start 157.375 98.375) (end 160 98.375) (width 0.2) (layer "F.Cu") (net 9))
 (segment (start 144.5 97.5) (end 147.5 97.5) (width 0.2) (layer "F.Cu") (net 9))
 (segment (start 148 97) (end 151 94) (width 0.2) (layer "F.Cu") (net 9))
 (segment (start 151 94) (end 154.5 94) (width 0.2) (layer "F.Cu") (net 9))
 (segment (start 155.5 95) (end 155.5 96.5) (width 0.2) (layer "F.Cu") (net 9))
 (segment (start 159.124999 101.624999) (end 159.125 101.625) (width 0.2) (layer "F.Cu") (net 30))
 (segment (start 159.125 101.625) (end 160 101.625) (width 0.2) (layer "F.Cu") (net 30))
 (segment (start 158 101.624999) (end 159.124999 101.624999) (width 0.2) (layer "F.Cu") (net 30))
 (via (at 158 101.624999) (size 0.6) (drill 0.3) (layers "F.Cu" "B.Cu") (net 30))
 (segment (start 158 101.624999) (end 146.624999 101.624999) (width 0.2) (layer "B.Cu") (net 30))
 (segment (start 143.23 98.23) (end 143.23 92.305) (width 0.2) (layer "B.Cu") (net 30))
 (segment (start 146.624999 101.624999) (end 143.23 98.23) (width 0.2) (layer "B.Cu") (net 30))
 (segment (start 161.326001 100.673999) (end 161.399 100.601) (width 0.2) (layer "F.Cu") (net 26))
 (segment (start 161.399 100.5) (end 161.399 90.498) (width 0.2) (layer "F.Cu") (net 26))
 (segment (start 161.399 100.601) (end 161.399 100.5) (width 0.2) (layer "F.Cu") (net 26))
 (segment (start 161.251 100.673999) (end 161.326001 100.673999) (width 0.2) (layer "F.Cu") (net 26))
 (segment (start 161.399 90.498) (end 159.401 88.5) (width 0.2) (layer "F.Cu") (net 26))
 (segment (start 160.949999 100.975) (end 161.251 100.673999) (width 0.2) (layer "F.Cu") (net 26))
 (segment (start 161.399 100.5) (end 161.399 99) (width 0.2) (layer "F.Cu") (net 26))
 (segment (start 160 100.975) (end 160.949999 100.975) (width 0.2) (layer "F.Cu") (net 26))
 (segment (start 158.075 102.925) (end 160 102.925) (width 0.2) (layer "F.Cu") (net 28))
 (segment (start 158 103) (end 158.075 102.925) (width 0.2) (layer "F.Cu") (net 28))
 (via (at 158 103) (size 0.6) (drill 0.3) (layers "F.Cu" "B.Cu") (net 28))
 (segment (start 145.5 103) (end 138.15 95.65) (width 0.2) (layer "B.Cu") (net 28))
 (segment (start 158 103) (end 145.5 103) (width 0.2) (layer "B.Cu") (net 28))
 (segment (start 138.15 95.65) (end 138.15 92.305) (width 0.2) (layer "B.Cu") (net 28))
 (segment (start 156.5 101.00513) (end 156.5 106.14) (width 0.2) (layer "F.Cu") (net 10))
 (segment (start 153 98.375) (end 153.86987 98.375) (width 0.2) (layer "F.Cu") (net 10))
 (segment (start 156.5 106.14) (end 158.74 108.38) (width 0.2) (layer "F.Cu") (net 10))
 (segment (start 153.86987 98.375) (end 156.5 101.00513) (width 0.2) (layer "F.Cu") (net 10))
 (segment (start 154.748943 101.20266) (end 155.101 101.554717) (width 0.2) (layer "F.Cu") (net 13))
 (segment (start 155.101 101.554717) (end 155.101 102.40466) (width 0.2) (layer "F.Cu") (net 13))
 (segment (start 153 100.325) (end 153.86987 100.325) (width 0.2) (layer "F.Cu") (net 13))
 (segment (start 155.101 104.399) (end 151.12 108.38) (width 0.2) (layer "F.Cu") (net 13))
 (segment (start 155.101 102.40466) (end 155.101 104.399) (width 0.2) (layer "F.Cu") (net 13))
 (segment (start 153.86987 100.325) (end 154.74753 101.20266) (width 0.2) (layer "F.Cu") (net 13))
 (segment (start 154.74753 101.20266) (end 154.748943 101.20266) (width 0.2) (layer "F.Cu") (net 13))
 (segment (start 151.401 103.68516) (end 151.401 101.624001) (width 0.2) (layer "F.Cu") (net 37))
 (segment (start 151.401 101.624001) (end 152.050001 100.975) (width 0.2) (layer "F.Cu") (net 37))
 (segment (start 152.050001 100.975) (end 153 100.975) (width 0.2) (layer "F.Cu") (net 37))
 (segment (start 153.86987 100.975) (end 153 100.975) (width 0.2) (layer "F.Cu") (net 37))
 (segment (start 139 106.5) (end 148.58616 106.5) (width 0.2) (layer "F.Cu") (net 37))
 (segment (start 148.58616 106.5) (end 151.401 103.68516) (width 0.2) (layer "F.Cu") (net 37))
 (via (at 139 106.5) (size 0.6) (drill 0.3) (layers "F.Cu" "B.Cu") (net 37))
 (segment (start 136.10104 113) (end 135.5 113) (width 0.2) (layer "B.Cu") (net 37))
 (segment (start 139 110.10104) (end 136.10104 113) (width 0.2) (layer "B.Cu") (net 37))
 (segment (start 139 106.5) (end 139 110.10104) (width 0.2) (layer "B.Cu") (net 37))
 (segment (start 158.575 103.575) (end 160 103.575) (width 0.2) (layer "F.Cu") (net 27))
 (segment (start 158.575 103.6) (end 158.575 103.575) (width 0.2) (layer "F.Cu") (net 27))
 (segment (start 157.1 103.6) (end 158.575 103.6) (width 0.2) (layer "F.Cu") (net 27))
 (via (at 157.1 103.6) (size 0.6) (drill 0.3) (layers "F.Cu" "B.Cu") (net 27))
 (segment (start 144.1 103.6) (end 135.61 95.11) (width 0.2) (layer "B.Cu") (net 27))
 (segment (start 135.61 95.11) (end 135.61 92.305) (width 0.2) (layer "B.Cu") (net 27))
 (segment (start 157.1 103.6) (end 144.1 103.6) (width 0.2) (layer "B.Cu") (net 27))
 (segment (start 155.502 106.538) (end 153.66 108.38) (width 0.2) (layer "F.Cu") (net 12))
 (segment (start 153.949999 99.675) (end 155.502 101.227001) (width 0.2) (layer "F.Cu") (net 12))
 (segment (start 153 99.675) (end 153.949999 99.675) (width 0.2) (layer "F.Cu") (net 12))
 (segment (start 155.502 101.227001) (end 155.502 106.538) (width 0.2) (layer "F.Cu") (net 12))
 (segment (start 157.309313 102.275) (end 160 102.275) (width 0.2) (layer "F.Cu") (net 29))
 (via (at 157.309313 102.275) (size 0.6) (drill 0.3) (layers "F.Cu" "B.Cu") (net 29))
 (segment (start 157.309313 102.275) (end 146.275 102.275) (width 0.2) (layer "B.Cu") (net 29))
 (segment (start 146.275 102.275) (end 140.69 96.69) (width 0.2) (layer "B.Cu") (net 29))
 (segment (start 140.69 96.69) (end 140.69 92.305) (width 0.2) (layer "B.Cu") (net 29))
 (segment (start 155.5 100.575001) (end 155.502771 100.575001) (width 0.2) (layer "F.Cu") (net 11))
 (segment (start 155.502771 100.575001) (end 156 101.07223) (width 0.2) (layer "F.Cu") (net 11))
 (segment (start 156 101.07223) (end 156 108.18) (width 0.2) (layer "F.Cu") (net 11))
 (segment (start 153.949999 99.025) (end 155.5 100.575001) (width 0.2) (layer "F.Cu") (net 11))
 (segment (start 156 108.18) (end 156.2 108.38) (width 0.2) (layer "F.Cu") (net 11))
 (segment (start 153 99.025) (end 153.949999 99.025) (width 0.2) (layer "F.Cu") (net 11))
 (segment (start 156.5 96.5) (end 157.075 97.075) (width 0.2) (layer "F.Cu") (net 24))
 (segment (start 157.075 97.075) (end 160 97.075) (width 0.2) (layer "F.Cu") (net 24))
 (via (at 156.5 96.5) (size 0.6) (drill 0.3) (layers "F.Cu" "B.Cu") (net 24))
 (segment (start 160.998 116.002) (end 154.5 122.5) (width 0.2) (layer "B.Cu") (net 24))
 (segment (start 160.998 101.7641) (end 160.998 116.002) (width 0.2) (layer "B.Cu") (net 24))
 (segment (start 155 82.5) (end 156.9 84.4) (width 0.2) (layer "B.Cu") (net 24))
 (segment (start 156.9 84.4) (end 156.9 97.6661) (width 0.2) (layer "B.Cu") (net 24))
 (segment (start 144 82.5) (end 155 82.5) (width 0.2) (layer "B.Cu") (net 24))
 (segment (start 139.5 78) (end 144 82.5) (width 0.2) (layer "B.Cu") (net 24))
 (segment (start 156.9 97.6661) (end 160.998 101.7641) (width 0.2) (layer "B.Cu") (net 24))
 (segment (start 158.5 97.725) (end 160 97.725) (width 0.2) (layer "F.Cu") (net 25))
 (via (at 158.5 97.725) (size 0.6) (drill 0.3) (layers "F.Cu" "B.Cu") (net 25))
 (segment (start 157.34853 97.5) (end 157.301 97.5) (width 0.2) (layer "B.Cu") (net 25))
 (segment (start 155 125) (end 152.5 122.5) (width 0.2) (layer "B.Cu") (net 25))
 (segment (start 141.5 78) (end 145 81.5) (width 0.2) (layer "B.Cu") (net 25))
 (segment (start 161.399 122.101) (end 158.5 125) (width 0.2) (layer "B.Cu") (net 25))
 (segment (start 155.5 81.5) (end 157.301 83.301) (width 0.2) (layer "B.Cu") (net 25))
 (segment (start 158.5 125) (end 155 125) (width 0.2) (layer "B.Cu") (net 25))
 (segment (start 161.399 101.598) (end 161.399 122.101) (width 0.2) (layer "B.Cu") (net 25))
 (segment (start 157.301 97.5) (end 161.399 101.598) (width 0.2) (layer "B.Cu") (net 25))
 (segment (start 157.301 83.301) (end 157.301 97.5) (width 0.2) (layer "B.Cu") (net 25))
 (segment (start 145 81.5) (end 155.5 81.5) (width 0.2) (layer "B.Cu") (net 25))
 (segment (start 157.57353 97.725) (end 157.34853 97.5) (width 0.2) (layer "B.Cu") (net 25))
 (segment (start 158.5 97.725) (end 157.57353 97.725) (width 0.2) (layer "B.Cu") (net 25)))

